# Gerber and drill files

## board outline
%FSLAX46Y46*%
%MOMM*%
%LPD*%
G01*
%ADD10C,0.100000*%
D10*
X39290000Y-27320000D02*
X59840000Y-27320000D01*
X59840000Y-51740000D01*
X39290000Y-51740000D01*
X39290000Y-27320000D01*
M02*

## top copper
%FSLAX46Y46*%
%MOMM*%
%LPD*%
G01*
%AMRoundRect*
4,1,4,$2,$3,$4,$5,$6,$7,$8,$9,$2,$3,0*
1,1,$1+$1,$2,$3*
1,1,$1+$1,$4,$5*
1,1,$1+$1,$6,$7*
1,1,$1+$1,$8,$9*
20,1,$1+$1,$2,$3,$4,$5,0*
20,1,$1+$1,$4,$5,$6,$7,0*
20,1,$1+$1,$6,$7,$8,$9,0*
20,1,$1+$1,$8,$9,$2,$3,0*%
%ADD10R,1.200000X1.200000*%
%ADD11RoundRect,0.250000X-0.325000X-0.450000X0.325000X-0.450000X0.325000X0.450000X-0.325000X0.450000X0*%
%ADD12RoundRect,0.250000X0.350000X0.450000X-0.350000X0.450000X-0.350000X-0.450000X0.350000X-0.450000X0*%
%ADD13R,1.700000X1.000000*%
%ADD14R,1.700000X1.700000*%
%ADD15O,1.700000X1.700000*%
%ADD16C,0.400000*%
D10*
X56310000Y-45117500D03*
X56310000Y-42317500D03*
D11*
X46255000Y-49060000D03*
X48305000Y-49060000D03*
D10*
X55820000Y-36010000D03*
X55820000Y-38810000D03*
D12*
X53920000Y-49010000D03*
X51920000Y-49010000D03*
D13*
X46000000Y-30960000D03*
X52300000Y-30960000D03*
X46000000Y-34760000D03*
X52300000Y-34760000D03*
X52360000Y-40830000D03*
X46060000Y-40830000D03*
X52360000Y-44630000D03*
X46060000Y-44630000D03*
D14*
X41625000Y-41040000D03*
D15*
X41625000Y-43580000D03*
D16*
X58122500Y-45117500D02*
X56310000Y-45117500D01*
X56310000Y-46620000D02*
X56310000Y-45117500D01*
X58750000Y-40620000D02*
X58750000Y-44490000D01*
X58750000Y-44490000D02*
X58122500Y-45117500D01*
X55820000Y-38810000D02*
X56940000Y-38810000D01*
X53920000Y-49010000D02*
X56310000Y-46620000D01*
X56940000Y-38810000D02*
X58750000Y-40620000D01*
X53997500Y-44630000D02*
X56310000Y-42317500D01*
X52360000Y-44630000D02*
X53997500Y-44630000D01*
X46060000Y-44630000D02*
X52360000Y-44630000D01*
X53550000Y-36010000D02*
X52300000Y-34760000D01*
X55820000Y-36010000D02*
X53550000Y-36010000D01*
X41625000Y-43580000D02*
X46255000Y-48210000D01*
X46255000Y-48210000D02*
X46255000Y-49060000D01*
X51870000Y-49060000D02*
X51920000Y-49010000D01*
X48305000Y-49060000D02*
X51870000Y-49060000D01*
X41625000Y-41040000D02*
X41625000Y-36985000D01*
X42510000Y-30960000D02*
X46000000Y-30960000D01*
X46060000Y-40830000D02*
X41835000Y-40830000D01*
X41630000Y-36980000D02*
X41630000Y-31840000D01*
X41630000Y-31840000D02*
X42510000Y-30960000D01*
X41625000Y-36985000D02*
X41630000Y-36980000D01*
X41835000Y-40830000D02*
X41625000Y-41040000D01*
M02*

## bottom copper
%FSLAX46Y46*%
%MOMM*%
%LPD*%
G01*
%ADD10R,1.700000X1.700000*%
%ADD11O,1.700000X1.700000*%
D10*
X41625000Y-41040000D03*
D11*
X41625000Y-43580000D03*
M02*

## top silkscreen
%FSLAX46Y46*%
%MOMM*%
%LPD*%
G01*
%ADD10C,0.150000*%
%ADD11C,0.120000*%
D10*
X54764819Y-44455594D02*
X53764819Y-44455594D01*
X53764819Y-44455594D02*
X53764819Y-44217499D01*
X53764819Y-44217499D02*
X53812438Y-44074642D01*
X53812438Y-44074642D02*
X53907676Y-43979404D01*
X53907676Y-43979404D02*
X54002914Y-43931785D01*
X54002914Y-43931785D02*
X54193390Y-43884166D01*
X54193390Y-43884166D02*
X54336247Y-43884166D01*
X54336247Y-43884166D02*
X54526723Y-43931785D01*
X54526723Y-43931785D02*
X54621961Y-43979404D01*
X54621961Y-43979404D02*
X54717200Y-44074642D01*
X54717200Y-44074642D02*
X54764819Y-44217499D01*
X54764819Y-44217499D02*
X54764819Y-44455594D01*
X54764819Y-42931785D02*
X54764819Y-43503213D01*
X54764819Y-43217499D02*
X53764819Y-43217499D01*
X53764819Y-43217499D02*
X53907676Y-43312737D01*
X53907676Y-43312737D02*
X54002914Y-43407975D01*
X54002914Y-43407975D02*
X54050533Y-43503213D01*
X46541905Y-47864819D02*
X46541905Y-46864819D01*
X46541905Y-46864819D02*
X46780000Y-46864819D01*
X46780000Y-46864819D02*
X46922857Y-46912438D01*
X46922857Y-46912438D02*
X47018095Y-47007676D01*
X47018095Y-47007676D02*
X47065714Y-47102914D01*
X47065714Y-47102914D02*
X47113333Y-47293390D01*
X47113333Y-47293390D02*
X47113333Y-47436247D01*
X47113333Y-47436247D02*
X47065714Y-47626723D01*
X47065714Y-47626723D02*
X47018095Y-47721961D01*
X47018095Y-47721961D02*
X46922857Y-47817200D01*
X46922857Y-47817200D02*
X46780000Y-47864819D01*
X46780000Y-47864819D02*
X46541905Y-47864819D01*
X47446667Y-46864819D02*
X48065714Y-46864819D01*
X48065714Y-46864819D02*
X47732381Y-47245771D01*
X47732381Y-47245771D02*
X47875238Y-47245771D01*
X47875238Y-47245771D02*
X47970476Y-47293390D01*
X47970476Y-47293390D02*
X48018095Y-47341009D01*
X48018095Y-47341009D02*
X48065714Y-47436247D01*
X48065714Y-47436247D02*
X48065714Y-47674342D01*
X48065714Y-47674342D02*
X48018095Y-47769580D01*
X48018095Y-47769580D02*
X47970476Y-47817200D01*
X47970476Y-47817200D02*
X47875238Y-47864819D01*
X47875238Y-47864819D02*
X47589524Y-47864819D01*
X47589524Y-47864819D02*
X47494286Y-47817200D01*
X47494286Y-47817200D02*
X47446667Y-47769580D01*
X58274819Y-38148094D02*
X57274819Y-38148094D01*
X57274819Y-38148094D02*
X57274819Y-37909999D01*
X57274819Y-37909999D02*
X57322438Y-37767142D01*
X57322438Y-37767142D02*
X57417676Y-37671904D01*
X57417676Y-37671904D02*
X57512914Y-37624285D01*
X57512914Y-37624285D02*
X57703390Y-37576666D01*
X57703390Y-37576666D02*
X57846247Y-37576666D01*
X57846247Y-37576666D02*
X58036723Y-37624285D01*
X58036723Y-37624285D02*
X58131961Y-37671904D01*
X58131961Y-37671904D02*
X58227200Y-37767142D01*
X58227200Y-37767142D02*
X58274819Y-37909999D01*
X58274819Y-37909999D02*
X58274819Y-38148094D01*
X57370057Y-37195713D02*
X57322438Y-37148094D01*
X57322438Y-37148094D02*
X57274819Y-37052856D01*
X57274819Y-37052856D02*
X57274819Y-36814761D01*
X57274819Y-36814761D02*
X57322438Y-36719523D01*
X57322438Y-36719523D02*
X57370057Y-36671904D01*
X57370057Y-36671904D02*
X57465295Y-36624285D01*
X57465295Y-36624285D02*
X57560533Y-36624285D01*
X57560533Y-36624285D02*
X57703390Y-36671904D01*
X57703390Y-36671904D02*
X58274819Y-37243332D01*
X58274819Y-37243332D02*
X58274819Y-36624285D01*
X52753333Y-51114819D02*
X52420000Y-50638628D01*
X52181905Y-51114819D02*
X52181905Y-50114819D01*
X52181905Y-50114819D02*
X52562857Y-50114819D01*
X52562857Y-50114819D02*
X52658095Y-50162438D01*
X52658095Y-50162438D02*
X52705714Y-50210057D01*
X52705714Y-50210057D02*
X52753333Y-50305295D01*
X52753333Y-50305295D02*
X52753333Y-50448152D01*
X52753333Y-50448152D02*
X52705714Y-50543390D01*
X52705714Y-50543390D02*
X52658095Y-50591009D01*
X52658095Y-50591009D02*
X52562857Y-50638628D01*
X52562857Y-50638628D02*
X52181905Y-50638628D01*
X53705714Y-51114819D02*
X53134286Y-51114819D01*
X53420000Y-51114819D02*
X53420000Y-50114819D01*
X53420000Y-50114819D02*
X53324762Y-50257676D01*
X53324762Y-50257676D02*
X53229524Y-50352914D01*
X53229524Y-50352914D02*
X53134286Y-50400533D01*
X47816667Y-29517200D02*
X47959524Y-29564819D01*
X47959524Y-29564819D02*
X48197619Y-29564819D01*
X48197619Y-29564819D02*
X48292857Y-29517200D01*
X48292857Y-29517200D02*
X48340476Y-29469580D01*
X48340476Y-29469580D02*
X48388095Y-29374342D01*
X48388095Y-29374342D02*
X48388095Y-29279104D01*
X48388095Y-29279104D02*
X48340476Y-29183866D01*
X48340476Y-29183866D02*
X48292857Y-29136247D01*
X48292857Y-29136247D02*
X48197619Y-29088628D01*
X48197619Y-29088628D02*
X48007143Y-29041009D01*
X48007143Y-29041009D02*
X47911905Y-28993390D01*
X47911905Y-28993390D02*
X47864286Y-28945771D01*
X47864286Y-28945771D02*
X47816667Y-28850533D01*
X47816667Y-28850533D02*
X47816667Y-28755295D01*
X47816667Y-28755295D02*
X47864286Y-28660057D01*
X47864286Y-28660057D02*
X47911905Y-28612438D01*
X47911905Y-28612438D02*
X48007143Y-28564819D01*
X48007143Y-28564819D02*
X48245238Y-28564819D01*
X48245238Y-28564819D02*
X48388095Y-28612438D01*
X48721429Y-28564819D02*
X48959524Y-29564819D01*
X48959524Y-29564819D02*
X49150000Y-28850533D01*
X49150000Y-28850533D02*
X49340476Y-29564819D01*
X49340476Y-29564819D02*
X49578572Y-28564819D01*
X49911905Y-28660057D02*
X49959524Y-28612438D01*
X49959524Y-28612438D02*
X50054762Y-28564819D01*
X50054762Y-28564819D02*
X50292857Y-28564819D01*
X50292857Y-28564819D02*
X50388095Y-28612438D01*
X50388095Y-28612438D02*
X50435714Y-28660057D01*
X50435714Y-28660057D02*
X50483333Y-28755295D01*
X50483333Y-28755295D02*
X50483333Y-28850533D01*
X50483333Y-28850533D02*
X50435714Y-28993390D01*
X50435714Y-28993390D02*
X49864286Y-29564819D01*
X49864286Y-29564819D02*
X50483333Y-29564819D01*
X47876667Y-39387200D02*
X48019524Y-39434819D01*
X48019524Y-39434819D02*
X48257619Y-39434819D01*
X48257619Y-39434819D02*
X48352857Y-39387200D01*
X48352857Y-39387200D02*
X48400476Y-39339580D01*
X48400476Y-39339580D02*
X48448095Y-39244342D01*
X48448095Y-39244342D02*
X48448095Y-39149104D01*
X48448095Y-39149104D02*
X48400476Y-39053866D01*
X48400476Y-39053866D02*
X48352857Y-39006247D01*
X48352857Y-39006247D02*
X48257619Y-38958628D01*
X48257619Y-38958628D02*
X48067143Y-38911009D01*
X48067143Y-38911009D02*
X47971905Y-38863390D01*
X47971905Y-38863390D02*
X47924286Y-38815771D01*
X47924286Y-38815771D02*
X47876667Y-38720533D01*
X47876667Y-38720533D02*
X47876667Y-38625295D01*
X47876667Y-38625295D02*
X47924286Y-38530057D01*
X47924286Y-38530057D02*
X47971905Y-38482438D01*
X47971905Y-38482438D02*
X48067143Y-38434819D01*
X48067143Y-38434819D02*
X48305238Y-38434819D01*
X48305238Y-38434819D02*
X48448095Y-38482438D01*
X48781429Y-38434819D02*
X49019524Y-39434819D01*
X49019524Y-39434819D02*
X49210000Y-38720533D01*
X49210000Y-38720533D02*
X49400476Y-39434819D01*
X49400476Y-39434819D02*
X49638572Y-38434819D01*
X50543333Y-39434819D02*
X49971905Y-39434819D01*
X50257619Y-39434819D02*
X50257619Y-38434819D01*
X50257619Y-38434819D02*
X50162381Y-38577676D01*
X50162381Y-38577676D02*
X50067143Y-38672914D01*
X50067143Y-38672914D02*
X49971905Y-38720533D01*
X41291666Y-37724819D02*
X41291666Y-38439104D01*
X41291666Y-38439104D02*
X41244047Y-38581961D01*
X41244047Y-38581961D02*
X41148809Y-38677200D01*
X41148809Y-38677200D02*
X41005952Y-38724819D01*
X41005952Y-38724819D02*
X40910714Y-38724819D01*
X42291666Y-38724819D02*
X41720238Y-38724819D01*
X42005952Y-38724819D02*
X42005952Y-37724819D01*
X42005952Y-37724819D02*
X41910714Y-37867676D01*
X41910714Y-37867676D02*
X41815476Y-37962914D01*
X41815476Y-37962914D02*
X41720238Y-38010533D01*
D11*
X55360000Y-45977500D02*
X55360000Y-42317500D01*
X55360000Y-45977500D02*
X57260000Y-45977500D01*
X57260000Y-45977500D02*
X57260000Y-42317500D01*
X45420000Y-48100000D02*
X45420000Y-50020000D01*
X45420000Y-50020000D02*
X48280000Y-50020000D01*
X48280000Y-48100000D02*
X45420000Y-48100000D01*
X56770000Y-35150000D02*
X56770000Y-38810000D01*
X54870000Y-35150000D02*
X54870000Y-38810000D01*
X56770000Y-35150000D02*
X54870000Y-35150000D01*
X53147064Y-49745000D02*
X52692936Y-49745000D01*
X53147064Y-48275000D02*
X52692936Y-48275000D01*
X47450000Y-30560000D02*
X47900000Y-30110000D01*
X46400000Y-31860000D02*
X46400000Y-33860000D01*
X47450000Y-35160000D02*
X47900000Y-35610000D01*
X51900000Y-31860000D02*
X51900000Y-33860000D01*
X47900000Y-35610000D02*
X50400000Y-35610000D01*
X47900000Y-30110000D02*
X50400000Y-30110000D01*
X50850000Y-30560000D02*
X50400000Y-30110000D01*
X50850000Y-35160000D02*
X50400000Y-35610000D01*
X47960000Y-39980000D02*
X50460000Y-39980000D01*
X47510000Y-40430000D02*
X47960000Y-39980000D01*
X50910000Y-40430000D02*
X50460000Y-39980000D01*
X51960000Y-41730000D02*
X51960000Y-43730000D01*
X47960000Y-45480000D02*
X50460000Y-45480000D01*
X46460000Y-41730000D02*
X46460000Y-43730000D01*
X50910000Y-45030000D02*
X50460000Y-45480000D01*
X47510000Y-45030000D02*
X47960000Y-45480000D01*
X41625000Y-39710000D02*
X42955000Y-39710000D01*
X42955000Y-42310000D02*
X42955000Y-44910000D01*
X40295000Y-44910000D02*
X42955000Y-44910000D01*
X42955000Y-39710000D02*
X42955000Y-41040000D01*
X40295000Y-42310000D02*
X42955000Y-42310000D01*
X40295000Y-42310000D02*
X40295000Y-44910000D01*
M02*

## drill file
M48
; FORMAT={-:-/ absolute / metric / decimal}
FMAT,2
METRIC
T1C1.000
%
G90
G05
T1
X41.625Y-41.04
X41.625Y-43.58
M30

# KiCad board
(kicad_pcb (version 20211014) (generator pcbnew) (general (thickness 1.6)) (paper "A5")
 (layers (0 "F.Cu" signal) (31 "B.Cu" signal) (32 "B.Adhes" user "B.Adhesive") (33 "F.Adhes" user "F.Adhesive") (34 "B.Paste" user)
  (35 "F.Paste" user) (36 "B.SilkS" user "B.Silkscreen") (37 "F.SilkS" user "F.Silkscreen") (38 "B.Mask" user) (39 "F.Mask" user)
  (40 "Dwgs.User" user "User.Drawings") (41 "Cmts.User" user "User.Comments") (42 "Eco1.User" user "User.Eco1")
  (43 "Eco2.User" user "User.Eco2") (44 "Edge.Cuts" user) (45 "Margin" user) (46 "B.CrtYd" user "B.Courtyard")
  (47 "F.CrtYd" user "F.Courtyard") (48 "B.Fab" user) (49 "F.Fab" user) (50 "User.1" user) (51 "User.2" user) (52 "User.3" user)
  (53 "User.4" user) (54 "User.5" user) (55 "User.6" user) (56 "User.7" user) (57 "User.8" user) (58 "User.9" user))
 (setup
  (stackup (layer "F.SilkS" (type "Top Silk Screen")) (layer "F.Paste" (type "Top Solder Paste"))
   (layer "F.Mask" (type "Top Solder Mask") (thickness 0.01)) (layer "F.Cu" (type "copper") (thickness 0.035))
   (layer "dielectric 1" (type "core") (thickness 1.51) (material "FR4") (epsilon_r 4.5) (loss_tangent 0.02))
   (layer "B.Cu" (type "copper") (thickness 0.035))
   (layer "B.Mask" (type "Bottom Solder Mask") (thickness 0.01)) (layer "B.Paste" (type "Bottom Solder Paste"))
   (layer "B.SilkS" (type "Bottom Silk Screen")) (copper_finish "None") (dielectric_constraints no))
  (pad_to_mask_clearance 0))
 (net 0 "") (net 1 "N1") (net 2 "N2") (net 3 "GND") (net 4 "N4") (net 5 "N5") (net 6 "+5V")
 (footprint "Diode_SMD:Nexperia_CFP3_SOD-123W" (layer "F.Cu") (at 56.31 43.7175 90)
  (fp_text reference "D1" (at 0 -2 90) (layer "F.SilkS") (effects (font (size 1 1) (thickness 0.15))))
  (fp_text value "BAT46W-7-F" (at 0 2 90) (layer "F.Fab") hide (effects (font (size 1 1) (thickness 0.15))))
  (fp_line (start -2.26 -0.95) (end 1.4 -0.95) (layer "F.SilkS") (width 0.12))
  (fp_line (start -2.26 -0.95) (end -2.26 0.95) (layer "F.SilkS") (width 0.12))
  (fp_line (start -2.26 0.95) (end 1.4 0.95) (layer "F.SilkS") (width 0.12))
  (pad "1" smd rect (at -1.4 0 90) (size 1.2 1.2) (layers "F.Cu" "F.Paste" "F.Mask") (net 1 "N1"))
  (pad "2" smd rect (at 1.4 0 90) (size 1.2 1.2) (layers "F.Cu" "F.Paste" "F.Mask") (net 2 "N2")))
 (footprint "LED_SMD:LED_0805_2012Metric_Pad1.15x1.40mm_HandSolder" (layer "F.Cu") (at 47.28 49.06)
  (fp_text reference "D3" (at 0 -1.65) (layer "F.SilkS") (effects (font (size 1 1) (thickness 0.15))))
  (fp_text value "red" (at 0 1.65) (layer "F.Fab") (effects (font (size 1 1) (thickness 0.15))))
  (fp_line (start -1.86 -0.96) (end -1.86 0.96) (layer "F.SilkS") (width 0.12))
  (fp_line (start -1.86 0.96) (end 1 0.96) (layer "F.SilkS") (width 0.12))
  (fp_line (start 1 -0.96) (end -1.86 -0.96) (layer "F.SilkS") (width 0.12))
  (pad "1" smd roundrect (at -1.025 0) (size 1.15 1.4) (layers "F.Cu" "F.Paste" "F.Mask") (roundrect_rratio 0.217391) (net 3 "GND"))
  (pad "2" smd roundrect (at 1.025 0) (size 1.15 1.4) (layers "F.Cu" "F.Paste" "F.Mask") (roundrect_rratio 0.217391) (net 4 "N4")))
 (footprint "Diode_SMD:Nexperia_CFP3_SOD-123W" (layer "F.Cu") (at 55.82 37.41 -90)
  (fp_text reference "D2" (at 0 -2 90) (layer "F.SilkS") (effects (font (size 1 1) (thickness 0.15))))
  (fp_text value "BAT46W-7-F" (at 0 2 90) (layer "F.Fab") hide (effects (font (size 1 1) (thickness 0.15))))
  (fp_line (start -2.26 -0.95) (end 1.4 -0.95) (layer "F.SilkS") (width 0.12))
  (fp_line (start -2.26 0.95) (end 1.4 0.95) (layer "F.SilkS") (width 0.12))
  (fp_line (start -2.26 -0.95) (end -2.26 0.95) (layer "F.SilkS") (width 0.12))
  (pad "1" smd rect (at -1.4 0 270) (size 1.2 1.2) (layers "F.Cu" "F.Paste" "F.Mask") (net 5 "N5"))
  (pad "2" smd rect (at 1.4 0 270) (size 1.2 1.2) (layers "F.Cu" "F.Paste" "F.Mask") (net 1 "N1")))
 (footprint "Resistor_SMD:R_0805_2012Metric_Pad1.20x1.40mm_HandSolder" (layer "F.Cu") (at 52.92 49.01 180)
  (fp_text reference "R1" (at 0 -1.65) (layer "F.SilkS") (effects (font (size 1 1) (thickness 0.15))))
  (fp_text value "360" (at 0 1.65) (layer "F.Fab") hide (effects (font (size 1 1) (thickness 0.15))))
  (fp_line (start -0.227064 -0.735) (end 0.227064 -0.735) (layer "F.SilkS") (width 0.12))
  (fp_line (start -0.227064 0.735) (end 0.227064 0.735) (layer "F.SilkS") (width 0.12))
  (pad "1" smd roundrect (at -1 0 180) (size 1.2 1.4) (layers "F.Cu" "F.Paste" "F.Mask") (roundrect_rratio 0.208333) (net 1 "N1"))
  (pad "2" smd roundrect (at 1 0 180) (size 1.2 1.4) (layers "F.Cu" "F.Paste" "F.Mask") (roundrect_rratio 0.208333) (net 4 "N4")))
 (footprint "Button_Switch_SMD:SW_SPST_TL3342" (layer "F.Cu") (at 49.15 32.86)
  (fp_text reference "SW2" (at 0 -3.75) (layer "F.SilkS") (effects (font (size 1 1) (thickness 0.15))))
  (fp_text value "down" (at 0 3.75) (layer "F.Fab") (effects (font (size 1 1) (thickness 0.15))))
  (fp_line (start -1.7 -2.3) (end -1.25 -2.75) (layer "F.SilkS") (width 0.12))
  (fp_line (start -2.75 -1) (end -2.75 1) (layer "F.SilkS") (width 0.12))
  (fp_line (start -1.7 2.3) (end -1.25 2.75) (layer "F.SilkS") (width 0.12))
  (fp_line (start 2.75 -1) (end 2.75 1) (layer "F.SilkS") (width 0.12))
  (fp_line (start -1.25 2.75) (end 1.25 2.75) (layer "F.SilkS") (width 0.12))
  (fp_line (start -1.25 -2.75) (end 1.25 -2.75) (layer "F.SilkS") (width 0.12))
  (fp_line (start 1.7 -2.3) (end 1.25 -2.75) (layer "F.SilkS") (width 0.12))
  (fp_line (start 1.7 2.3) (end 1.25 2.75) (layer "F.SilkS") (width 0.12))
  (pad "1" smd rect (at -3.15 -1.9) (size 1.7 1) (layers "F.Cu" "F.Paste" "F.Mask") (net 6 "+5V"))
  (pad "1" smd rect (at 3.15 -1.9) (size 1.7 1) (layers "F.Cu" "F.Paste" "F.Mask") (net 6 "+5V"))
  (pad "2" smd rect (at -3.15 1.9) (size 1.7 1) (layers "F.Cu" "F.Paste" "F.Mask") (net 5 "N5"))
  (pad "2" smd rect (at 3.15 1.9) (size 1.7 1) (layers "F.Cu" "F.Paste" "F.Mask") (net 5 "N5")))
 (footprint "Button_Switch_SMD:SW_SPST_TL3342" (layer "F.Cu") (at 49.21 42.73)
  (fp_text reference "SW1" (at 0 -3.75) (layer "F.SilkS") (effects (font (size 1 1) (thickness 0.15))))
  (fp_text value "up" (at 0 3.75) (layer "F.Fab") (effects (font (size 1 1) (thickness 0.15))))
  (fp_line (start -1.25 -2.75) (end 1.25 -2.75) (layer "F.SilkS") (width 0.12))
  (fp_line (start -1.7 -2.3) (end -1.25 -2.75) (layer "F.SilkS") (width 0.12))
  (fp_line (start 1.7 -2.3) (end 1.25 -2.75) (layer "F.SilkS") (width 0.12))
  (fp_line (start 2.75 -1) (end 2.75 1) (layer "F.SilkS") (width 0.12))
  (fp_line (start -1.25 2.75) (end 1.25 2.75) (layer "F.SilkS") (width 0.12))
  (fp_line (start -2.75 -1) (end -2.75 1) (layer "F.SilkS") (width 0.12))
  (fp_line (start 1.7 2.3) (end 1.25 2.75) (layer "F.SilkS") (width 0.12))
  (fp_line (start -1.7 2.3) (end -1.25 2.75) (layer "F.SilkS") (width 0.12))
  (pad "1" smd rect (at 3.15 -1.9) (size 1.7 1) (layers "F.Cu" "F.Paste" "F.Mask") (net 6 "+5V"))
  (pad "1" smd rect (at -3.15 -1.9) (size 1.7 1) (layers "F.Cu" "F.Paste" "F.Mask") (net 6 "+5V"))
  (pad "2" smd rect (at 3.15 1.9) (size 1.7 1) (layers "F.Cu" "F.Paste" "F.Mask") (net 2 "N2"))
  (pad "2" smd rect (at -3.15 1.9) (size 1.7 1) (layers "F.Cu" "F.Paste" "F.Mask") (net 2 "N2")))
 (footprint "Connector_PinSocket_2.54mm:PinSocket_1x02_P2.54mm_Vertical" (layer "F.Cu") (at 41.625 41.04)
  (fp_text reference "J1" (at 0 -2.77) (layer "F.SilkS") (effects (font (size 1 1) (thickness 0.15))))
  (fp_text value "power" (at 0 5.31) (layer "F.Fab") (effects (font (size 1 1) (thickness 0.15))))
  (fp_line (start 0 -1.33) (end 1.33 -1.33) (layer "F.SilkS") (width 0.12))
  (fp_line (start 1.33 1.27) (end 1.33 3.87) (layer "F.SilkS") (width 0.12))
  (fp_line (start -1.33 3.87) (end 1.33 3.87) (layer "F.SilkS") (width 0.12))
  (fp_line (start 1.33 -1.33) (end 1.33 0) (layer "F.SilkS") (width 0.12))
  (fp_line (start -1.33 1.27) (end 1.33 1.27) (layer "F.SilkS") (width 0.12))
  (fp_line (start -1.33 1.27) (end -1.33 3.87) (layer "F.SilkS") (width 0.12))
  (pad "1" thru_hole rect (at 0 0) (size 1.7 1.7) (drill 1) (layers *.Cu *.Mask) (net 6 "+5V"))
  (pad "2" thru_hole oval (at 0 2.54) (size 1.7 1.7) (drill 1) (layers *.Cu *.Mask) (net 3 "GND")))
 (gr_rect (start 39.29 27.32) (end 59.84 51.74) (layer "Edge.Cuts") (width 0.1) (fill none))
 (segment (start 58.1225 45.1175) (end 56.31 45.1175) (width 0.4) (layer "F.Cu") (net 1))
 (segment (start 56.31 46.62) (end 56.31 45.1175) (width 0.4) (layer "F.Cu") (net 1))
 (segment (start 58.75 40.62) (end 58.75 44.49) (width 0.4) (layer "F.Cu") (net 1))
 (segment (start 58.75 44.49) (end 58.1225 45.1175) (width 0.4) (layer "F.Cu") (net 1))
 (segment (start 55.82 38.81) (end 56.94 38.81) (width 0.4) (layer "F.Cu") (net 1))
 (segment (start 53.92 49.01) (end 56.31 46.62) (width 0.4) (layer "F.Cu") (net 1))
 (segment (start 56.94 38.81) (end 58.75 40.62) (width 0.4) (layer "F.Cu") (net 1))
 (segment (start 53.9975 44.63) (end 56.31 42.3175) (width 0.4) (layer "F.Cu") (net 2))
 (segment (start 52.36 44.63) (end 53.9975 44.63) (width 0.4) (layer "F.Cu") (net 2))
 (segment (start 46.06 44.63) (end 52.36 44.63) (width 0.4) (layer "F.Cu") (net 2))
 (segment (start 53.55 36.01) (end 52.3 34.76) (width 0.4) (layer "F.Cu") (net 5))
 (segment (start 55.82 36.01) (end 53.55 36.01) (width 0.4) (layer "F.Cu") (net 5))
 (segment (start 41.625 43.58) (end 46.255 48.21) (width 0.4) (layer "F.Cu") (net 3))
 (segment (start 46.255 48.21) (end 46.255 49.06) (width 0.4) (layer "F.Cu") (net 3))
 (segment (start 51.87 49.06) (end 51.92 49.01) (width 0.4) (layer "F.Cu") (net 4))
 (segment (start 48.305 49.06) (end 51.87 49.06) (width 0.4) (layer "F.Cu") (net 4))
 (segment (start 41.625 41.04) (end 41.625 36.985) (width 0.4) (layer "F.Cu") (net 6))
 (segment (start 42.51 30.96) (end 46 30.96) (width 0.4) (layer "F.Cu") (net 6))
 (segment (start 46.06 40.83) (end 41.835 40.83) (width 0.4) (layer "F.Cu") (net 6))
 (segment (start 41.63 36.98) (end 41.63 31.84) (width 0.4) (layer "F.Cu") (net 6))
 (segment (start 41.63 31.84) (end 42.51 30.96) (width 0.4) (layer "F.Cu") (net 6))
 (segment (start 41.625 36.985) (end 41.63 36.98) (width 0.4) (layer "F.Cu") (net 6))
 (segment (start 41.835 40.83) (end 41.625 41.04) (width 0.4) (layer "F.Cu") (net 6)))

